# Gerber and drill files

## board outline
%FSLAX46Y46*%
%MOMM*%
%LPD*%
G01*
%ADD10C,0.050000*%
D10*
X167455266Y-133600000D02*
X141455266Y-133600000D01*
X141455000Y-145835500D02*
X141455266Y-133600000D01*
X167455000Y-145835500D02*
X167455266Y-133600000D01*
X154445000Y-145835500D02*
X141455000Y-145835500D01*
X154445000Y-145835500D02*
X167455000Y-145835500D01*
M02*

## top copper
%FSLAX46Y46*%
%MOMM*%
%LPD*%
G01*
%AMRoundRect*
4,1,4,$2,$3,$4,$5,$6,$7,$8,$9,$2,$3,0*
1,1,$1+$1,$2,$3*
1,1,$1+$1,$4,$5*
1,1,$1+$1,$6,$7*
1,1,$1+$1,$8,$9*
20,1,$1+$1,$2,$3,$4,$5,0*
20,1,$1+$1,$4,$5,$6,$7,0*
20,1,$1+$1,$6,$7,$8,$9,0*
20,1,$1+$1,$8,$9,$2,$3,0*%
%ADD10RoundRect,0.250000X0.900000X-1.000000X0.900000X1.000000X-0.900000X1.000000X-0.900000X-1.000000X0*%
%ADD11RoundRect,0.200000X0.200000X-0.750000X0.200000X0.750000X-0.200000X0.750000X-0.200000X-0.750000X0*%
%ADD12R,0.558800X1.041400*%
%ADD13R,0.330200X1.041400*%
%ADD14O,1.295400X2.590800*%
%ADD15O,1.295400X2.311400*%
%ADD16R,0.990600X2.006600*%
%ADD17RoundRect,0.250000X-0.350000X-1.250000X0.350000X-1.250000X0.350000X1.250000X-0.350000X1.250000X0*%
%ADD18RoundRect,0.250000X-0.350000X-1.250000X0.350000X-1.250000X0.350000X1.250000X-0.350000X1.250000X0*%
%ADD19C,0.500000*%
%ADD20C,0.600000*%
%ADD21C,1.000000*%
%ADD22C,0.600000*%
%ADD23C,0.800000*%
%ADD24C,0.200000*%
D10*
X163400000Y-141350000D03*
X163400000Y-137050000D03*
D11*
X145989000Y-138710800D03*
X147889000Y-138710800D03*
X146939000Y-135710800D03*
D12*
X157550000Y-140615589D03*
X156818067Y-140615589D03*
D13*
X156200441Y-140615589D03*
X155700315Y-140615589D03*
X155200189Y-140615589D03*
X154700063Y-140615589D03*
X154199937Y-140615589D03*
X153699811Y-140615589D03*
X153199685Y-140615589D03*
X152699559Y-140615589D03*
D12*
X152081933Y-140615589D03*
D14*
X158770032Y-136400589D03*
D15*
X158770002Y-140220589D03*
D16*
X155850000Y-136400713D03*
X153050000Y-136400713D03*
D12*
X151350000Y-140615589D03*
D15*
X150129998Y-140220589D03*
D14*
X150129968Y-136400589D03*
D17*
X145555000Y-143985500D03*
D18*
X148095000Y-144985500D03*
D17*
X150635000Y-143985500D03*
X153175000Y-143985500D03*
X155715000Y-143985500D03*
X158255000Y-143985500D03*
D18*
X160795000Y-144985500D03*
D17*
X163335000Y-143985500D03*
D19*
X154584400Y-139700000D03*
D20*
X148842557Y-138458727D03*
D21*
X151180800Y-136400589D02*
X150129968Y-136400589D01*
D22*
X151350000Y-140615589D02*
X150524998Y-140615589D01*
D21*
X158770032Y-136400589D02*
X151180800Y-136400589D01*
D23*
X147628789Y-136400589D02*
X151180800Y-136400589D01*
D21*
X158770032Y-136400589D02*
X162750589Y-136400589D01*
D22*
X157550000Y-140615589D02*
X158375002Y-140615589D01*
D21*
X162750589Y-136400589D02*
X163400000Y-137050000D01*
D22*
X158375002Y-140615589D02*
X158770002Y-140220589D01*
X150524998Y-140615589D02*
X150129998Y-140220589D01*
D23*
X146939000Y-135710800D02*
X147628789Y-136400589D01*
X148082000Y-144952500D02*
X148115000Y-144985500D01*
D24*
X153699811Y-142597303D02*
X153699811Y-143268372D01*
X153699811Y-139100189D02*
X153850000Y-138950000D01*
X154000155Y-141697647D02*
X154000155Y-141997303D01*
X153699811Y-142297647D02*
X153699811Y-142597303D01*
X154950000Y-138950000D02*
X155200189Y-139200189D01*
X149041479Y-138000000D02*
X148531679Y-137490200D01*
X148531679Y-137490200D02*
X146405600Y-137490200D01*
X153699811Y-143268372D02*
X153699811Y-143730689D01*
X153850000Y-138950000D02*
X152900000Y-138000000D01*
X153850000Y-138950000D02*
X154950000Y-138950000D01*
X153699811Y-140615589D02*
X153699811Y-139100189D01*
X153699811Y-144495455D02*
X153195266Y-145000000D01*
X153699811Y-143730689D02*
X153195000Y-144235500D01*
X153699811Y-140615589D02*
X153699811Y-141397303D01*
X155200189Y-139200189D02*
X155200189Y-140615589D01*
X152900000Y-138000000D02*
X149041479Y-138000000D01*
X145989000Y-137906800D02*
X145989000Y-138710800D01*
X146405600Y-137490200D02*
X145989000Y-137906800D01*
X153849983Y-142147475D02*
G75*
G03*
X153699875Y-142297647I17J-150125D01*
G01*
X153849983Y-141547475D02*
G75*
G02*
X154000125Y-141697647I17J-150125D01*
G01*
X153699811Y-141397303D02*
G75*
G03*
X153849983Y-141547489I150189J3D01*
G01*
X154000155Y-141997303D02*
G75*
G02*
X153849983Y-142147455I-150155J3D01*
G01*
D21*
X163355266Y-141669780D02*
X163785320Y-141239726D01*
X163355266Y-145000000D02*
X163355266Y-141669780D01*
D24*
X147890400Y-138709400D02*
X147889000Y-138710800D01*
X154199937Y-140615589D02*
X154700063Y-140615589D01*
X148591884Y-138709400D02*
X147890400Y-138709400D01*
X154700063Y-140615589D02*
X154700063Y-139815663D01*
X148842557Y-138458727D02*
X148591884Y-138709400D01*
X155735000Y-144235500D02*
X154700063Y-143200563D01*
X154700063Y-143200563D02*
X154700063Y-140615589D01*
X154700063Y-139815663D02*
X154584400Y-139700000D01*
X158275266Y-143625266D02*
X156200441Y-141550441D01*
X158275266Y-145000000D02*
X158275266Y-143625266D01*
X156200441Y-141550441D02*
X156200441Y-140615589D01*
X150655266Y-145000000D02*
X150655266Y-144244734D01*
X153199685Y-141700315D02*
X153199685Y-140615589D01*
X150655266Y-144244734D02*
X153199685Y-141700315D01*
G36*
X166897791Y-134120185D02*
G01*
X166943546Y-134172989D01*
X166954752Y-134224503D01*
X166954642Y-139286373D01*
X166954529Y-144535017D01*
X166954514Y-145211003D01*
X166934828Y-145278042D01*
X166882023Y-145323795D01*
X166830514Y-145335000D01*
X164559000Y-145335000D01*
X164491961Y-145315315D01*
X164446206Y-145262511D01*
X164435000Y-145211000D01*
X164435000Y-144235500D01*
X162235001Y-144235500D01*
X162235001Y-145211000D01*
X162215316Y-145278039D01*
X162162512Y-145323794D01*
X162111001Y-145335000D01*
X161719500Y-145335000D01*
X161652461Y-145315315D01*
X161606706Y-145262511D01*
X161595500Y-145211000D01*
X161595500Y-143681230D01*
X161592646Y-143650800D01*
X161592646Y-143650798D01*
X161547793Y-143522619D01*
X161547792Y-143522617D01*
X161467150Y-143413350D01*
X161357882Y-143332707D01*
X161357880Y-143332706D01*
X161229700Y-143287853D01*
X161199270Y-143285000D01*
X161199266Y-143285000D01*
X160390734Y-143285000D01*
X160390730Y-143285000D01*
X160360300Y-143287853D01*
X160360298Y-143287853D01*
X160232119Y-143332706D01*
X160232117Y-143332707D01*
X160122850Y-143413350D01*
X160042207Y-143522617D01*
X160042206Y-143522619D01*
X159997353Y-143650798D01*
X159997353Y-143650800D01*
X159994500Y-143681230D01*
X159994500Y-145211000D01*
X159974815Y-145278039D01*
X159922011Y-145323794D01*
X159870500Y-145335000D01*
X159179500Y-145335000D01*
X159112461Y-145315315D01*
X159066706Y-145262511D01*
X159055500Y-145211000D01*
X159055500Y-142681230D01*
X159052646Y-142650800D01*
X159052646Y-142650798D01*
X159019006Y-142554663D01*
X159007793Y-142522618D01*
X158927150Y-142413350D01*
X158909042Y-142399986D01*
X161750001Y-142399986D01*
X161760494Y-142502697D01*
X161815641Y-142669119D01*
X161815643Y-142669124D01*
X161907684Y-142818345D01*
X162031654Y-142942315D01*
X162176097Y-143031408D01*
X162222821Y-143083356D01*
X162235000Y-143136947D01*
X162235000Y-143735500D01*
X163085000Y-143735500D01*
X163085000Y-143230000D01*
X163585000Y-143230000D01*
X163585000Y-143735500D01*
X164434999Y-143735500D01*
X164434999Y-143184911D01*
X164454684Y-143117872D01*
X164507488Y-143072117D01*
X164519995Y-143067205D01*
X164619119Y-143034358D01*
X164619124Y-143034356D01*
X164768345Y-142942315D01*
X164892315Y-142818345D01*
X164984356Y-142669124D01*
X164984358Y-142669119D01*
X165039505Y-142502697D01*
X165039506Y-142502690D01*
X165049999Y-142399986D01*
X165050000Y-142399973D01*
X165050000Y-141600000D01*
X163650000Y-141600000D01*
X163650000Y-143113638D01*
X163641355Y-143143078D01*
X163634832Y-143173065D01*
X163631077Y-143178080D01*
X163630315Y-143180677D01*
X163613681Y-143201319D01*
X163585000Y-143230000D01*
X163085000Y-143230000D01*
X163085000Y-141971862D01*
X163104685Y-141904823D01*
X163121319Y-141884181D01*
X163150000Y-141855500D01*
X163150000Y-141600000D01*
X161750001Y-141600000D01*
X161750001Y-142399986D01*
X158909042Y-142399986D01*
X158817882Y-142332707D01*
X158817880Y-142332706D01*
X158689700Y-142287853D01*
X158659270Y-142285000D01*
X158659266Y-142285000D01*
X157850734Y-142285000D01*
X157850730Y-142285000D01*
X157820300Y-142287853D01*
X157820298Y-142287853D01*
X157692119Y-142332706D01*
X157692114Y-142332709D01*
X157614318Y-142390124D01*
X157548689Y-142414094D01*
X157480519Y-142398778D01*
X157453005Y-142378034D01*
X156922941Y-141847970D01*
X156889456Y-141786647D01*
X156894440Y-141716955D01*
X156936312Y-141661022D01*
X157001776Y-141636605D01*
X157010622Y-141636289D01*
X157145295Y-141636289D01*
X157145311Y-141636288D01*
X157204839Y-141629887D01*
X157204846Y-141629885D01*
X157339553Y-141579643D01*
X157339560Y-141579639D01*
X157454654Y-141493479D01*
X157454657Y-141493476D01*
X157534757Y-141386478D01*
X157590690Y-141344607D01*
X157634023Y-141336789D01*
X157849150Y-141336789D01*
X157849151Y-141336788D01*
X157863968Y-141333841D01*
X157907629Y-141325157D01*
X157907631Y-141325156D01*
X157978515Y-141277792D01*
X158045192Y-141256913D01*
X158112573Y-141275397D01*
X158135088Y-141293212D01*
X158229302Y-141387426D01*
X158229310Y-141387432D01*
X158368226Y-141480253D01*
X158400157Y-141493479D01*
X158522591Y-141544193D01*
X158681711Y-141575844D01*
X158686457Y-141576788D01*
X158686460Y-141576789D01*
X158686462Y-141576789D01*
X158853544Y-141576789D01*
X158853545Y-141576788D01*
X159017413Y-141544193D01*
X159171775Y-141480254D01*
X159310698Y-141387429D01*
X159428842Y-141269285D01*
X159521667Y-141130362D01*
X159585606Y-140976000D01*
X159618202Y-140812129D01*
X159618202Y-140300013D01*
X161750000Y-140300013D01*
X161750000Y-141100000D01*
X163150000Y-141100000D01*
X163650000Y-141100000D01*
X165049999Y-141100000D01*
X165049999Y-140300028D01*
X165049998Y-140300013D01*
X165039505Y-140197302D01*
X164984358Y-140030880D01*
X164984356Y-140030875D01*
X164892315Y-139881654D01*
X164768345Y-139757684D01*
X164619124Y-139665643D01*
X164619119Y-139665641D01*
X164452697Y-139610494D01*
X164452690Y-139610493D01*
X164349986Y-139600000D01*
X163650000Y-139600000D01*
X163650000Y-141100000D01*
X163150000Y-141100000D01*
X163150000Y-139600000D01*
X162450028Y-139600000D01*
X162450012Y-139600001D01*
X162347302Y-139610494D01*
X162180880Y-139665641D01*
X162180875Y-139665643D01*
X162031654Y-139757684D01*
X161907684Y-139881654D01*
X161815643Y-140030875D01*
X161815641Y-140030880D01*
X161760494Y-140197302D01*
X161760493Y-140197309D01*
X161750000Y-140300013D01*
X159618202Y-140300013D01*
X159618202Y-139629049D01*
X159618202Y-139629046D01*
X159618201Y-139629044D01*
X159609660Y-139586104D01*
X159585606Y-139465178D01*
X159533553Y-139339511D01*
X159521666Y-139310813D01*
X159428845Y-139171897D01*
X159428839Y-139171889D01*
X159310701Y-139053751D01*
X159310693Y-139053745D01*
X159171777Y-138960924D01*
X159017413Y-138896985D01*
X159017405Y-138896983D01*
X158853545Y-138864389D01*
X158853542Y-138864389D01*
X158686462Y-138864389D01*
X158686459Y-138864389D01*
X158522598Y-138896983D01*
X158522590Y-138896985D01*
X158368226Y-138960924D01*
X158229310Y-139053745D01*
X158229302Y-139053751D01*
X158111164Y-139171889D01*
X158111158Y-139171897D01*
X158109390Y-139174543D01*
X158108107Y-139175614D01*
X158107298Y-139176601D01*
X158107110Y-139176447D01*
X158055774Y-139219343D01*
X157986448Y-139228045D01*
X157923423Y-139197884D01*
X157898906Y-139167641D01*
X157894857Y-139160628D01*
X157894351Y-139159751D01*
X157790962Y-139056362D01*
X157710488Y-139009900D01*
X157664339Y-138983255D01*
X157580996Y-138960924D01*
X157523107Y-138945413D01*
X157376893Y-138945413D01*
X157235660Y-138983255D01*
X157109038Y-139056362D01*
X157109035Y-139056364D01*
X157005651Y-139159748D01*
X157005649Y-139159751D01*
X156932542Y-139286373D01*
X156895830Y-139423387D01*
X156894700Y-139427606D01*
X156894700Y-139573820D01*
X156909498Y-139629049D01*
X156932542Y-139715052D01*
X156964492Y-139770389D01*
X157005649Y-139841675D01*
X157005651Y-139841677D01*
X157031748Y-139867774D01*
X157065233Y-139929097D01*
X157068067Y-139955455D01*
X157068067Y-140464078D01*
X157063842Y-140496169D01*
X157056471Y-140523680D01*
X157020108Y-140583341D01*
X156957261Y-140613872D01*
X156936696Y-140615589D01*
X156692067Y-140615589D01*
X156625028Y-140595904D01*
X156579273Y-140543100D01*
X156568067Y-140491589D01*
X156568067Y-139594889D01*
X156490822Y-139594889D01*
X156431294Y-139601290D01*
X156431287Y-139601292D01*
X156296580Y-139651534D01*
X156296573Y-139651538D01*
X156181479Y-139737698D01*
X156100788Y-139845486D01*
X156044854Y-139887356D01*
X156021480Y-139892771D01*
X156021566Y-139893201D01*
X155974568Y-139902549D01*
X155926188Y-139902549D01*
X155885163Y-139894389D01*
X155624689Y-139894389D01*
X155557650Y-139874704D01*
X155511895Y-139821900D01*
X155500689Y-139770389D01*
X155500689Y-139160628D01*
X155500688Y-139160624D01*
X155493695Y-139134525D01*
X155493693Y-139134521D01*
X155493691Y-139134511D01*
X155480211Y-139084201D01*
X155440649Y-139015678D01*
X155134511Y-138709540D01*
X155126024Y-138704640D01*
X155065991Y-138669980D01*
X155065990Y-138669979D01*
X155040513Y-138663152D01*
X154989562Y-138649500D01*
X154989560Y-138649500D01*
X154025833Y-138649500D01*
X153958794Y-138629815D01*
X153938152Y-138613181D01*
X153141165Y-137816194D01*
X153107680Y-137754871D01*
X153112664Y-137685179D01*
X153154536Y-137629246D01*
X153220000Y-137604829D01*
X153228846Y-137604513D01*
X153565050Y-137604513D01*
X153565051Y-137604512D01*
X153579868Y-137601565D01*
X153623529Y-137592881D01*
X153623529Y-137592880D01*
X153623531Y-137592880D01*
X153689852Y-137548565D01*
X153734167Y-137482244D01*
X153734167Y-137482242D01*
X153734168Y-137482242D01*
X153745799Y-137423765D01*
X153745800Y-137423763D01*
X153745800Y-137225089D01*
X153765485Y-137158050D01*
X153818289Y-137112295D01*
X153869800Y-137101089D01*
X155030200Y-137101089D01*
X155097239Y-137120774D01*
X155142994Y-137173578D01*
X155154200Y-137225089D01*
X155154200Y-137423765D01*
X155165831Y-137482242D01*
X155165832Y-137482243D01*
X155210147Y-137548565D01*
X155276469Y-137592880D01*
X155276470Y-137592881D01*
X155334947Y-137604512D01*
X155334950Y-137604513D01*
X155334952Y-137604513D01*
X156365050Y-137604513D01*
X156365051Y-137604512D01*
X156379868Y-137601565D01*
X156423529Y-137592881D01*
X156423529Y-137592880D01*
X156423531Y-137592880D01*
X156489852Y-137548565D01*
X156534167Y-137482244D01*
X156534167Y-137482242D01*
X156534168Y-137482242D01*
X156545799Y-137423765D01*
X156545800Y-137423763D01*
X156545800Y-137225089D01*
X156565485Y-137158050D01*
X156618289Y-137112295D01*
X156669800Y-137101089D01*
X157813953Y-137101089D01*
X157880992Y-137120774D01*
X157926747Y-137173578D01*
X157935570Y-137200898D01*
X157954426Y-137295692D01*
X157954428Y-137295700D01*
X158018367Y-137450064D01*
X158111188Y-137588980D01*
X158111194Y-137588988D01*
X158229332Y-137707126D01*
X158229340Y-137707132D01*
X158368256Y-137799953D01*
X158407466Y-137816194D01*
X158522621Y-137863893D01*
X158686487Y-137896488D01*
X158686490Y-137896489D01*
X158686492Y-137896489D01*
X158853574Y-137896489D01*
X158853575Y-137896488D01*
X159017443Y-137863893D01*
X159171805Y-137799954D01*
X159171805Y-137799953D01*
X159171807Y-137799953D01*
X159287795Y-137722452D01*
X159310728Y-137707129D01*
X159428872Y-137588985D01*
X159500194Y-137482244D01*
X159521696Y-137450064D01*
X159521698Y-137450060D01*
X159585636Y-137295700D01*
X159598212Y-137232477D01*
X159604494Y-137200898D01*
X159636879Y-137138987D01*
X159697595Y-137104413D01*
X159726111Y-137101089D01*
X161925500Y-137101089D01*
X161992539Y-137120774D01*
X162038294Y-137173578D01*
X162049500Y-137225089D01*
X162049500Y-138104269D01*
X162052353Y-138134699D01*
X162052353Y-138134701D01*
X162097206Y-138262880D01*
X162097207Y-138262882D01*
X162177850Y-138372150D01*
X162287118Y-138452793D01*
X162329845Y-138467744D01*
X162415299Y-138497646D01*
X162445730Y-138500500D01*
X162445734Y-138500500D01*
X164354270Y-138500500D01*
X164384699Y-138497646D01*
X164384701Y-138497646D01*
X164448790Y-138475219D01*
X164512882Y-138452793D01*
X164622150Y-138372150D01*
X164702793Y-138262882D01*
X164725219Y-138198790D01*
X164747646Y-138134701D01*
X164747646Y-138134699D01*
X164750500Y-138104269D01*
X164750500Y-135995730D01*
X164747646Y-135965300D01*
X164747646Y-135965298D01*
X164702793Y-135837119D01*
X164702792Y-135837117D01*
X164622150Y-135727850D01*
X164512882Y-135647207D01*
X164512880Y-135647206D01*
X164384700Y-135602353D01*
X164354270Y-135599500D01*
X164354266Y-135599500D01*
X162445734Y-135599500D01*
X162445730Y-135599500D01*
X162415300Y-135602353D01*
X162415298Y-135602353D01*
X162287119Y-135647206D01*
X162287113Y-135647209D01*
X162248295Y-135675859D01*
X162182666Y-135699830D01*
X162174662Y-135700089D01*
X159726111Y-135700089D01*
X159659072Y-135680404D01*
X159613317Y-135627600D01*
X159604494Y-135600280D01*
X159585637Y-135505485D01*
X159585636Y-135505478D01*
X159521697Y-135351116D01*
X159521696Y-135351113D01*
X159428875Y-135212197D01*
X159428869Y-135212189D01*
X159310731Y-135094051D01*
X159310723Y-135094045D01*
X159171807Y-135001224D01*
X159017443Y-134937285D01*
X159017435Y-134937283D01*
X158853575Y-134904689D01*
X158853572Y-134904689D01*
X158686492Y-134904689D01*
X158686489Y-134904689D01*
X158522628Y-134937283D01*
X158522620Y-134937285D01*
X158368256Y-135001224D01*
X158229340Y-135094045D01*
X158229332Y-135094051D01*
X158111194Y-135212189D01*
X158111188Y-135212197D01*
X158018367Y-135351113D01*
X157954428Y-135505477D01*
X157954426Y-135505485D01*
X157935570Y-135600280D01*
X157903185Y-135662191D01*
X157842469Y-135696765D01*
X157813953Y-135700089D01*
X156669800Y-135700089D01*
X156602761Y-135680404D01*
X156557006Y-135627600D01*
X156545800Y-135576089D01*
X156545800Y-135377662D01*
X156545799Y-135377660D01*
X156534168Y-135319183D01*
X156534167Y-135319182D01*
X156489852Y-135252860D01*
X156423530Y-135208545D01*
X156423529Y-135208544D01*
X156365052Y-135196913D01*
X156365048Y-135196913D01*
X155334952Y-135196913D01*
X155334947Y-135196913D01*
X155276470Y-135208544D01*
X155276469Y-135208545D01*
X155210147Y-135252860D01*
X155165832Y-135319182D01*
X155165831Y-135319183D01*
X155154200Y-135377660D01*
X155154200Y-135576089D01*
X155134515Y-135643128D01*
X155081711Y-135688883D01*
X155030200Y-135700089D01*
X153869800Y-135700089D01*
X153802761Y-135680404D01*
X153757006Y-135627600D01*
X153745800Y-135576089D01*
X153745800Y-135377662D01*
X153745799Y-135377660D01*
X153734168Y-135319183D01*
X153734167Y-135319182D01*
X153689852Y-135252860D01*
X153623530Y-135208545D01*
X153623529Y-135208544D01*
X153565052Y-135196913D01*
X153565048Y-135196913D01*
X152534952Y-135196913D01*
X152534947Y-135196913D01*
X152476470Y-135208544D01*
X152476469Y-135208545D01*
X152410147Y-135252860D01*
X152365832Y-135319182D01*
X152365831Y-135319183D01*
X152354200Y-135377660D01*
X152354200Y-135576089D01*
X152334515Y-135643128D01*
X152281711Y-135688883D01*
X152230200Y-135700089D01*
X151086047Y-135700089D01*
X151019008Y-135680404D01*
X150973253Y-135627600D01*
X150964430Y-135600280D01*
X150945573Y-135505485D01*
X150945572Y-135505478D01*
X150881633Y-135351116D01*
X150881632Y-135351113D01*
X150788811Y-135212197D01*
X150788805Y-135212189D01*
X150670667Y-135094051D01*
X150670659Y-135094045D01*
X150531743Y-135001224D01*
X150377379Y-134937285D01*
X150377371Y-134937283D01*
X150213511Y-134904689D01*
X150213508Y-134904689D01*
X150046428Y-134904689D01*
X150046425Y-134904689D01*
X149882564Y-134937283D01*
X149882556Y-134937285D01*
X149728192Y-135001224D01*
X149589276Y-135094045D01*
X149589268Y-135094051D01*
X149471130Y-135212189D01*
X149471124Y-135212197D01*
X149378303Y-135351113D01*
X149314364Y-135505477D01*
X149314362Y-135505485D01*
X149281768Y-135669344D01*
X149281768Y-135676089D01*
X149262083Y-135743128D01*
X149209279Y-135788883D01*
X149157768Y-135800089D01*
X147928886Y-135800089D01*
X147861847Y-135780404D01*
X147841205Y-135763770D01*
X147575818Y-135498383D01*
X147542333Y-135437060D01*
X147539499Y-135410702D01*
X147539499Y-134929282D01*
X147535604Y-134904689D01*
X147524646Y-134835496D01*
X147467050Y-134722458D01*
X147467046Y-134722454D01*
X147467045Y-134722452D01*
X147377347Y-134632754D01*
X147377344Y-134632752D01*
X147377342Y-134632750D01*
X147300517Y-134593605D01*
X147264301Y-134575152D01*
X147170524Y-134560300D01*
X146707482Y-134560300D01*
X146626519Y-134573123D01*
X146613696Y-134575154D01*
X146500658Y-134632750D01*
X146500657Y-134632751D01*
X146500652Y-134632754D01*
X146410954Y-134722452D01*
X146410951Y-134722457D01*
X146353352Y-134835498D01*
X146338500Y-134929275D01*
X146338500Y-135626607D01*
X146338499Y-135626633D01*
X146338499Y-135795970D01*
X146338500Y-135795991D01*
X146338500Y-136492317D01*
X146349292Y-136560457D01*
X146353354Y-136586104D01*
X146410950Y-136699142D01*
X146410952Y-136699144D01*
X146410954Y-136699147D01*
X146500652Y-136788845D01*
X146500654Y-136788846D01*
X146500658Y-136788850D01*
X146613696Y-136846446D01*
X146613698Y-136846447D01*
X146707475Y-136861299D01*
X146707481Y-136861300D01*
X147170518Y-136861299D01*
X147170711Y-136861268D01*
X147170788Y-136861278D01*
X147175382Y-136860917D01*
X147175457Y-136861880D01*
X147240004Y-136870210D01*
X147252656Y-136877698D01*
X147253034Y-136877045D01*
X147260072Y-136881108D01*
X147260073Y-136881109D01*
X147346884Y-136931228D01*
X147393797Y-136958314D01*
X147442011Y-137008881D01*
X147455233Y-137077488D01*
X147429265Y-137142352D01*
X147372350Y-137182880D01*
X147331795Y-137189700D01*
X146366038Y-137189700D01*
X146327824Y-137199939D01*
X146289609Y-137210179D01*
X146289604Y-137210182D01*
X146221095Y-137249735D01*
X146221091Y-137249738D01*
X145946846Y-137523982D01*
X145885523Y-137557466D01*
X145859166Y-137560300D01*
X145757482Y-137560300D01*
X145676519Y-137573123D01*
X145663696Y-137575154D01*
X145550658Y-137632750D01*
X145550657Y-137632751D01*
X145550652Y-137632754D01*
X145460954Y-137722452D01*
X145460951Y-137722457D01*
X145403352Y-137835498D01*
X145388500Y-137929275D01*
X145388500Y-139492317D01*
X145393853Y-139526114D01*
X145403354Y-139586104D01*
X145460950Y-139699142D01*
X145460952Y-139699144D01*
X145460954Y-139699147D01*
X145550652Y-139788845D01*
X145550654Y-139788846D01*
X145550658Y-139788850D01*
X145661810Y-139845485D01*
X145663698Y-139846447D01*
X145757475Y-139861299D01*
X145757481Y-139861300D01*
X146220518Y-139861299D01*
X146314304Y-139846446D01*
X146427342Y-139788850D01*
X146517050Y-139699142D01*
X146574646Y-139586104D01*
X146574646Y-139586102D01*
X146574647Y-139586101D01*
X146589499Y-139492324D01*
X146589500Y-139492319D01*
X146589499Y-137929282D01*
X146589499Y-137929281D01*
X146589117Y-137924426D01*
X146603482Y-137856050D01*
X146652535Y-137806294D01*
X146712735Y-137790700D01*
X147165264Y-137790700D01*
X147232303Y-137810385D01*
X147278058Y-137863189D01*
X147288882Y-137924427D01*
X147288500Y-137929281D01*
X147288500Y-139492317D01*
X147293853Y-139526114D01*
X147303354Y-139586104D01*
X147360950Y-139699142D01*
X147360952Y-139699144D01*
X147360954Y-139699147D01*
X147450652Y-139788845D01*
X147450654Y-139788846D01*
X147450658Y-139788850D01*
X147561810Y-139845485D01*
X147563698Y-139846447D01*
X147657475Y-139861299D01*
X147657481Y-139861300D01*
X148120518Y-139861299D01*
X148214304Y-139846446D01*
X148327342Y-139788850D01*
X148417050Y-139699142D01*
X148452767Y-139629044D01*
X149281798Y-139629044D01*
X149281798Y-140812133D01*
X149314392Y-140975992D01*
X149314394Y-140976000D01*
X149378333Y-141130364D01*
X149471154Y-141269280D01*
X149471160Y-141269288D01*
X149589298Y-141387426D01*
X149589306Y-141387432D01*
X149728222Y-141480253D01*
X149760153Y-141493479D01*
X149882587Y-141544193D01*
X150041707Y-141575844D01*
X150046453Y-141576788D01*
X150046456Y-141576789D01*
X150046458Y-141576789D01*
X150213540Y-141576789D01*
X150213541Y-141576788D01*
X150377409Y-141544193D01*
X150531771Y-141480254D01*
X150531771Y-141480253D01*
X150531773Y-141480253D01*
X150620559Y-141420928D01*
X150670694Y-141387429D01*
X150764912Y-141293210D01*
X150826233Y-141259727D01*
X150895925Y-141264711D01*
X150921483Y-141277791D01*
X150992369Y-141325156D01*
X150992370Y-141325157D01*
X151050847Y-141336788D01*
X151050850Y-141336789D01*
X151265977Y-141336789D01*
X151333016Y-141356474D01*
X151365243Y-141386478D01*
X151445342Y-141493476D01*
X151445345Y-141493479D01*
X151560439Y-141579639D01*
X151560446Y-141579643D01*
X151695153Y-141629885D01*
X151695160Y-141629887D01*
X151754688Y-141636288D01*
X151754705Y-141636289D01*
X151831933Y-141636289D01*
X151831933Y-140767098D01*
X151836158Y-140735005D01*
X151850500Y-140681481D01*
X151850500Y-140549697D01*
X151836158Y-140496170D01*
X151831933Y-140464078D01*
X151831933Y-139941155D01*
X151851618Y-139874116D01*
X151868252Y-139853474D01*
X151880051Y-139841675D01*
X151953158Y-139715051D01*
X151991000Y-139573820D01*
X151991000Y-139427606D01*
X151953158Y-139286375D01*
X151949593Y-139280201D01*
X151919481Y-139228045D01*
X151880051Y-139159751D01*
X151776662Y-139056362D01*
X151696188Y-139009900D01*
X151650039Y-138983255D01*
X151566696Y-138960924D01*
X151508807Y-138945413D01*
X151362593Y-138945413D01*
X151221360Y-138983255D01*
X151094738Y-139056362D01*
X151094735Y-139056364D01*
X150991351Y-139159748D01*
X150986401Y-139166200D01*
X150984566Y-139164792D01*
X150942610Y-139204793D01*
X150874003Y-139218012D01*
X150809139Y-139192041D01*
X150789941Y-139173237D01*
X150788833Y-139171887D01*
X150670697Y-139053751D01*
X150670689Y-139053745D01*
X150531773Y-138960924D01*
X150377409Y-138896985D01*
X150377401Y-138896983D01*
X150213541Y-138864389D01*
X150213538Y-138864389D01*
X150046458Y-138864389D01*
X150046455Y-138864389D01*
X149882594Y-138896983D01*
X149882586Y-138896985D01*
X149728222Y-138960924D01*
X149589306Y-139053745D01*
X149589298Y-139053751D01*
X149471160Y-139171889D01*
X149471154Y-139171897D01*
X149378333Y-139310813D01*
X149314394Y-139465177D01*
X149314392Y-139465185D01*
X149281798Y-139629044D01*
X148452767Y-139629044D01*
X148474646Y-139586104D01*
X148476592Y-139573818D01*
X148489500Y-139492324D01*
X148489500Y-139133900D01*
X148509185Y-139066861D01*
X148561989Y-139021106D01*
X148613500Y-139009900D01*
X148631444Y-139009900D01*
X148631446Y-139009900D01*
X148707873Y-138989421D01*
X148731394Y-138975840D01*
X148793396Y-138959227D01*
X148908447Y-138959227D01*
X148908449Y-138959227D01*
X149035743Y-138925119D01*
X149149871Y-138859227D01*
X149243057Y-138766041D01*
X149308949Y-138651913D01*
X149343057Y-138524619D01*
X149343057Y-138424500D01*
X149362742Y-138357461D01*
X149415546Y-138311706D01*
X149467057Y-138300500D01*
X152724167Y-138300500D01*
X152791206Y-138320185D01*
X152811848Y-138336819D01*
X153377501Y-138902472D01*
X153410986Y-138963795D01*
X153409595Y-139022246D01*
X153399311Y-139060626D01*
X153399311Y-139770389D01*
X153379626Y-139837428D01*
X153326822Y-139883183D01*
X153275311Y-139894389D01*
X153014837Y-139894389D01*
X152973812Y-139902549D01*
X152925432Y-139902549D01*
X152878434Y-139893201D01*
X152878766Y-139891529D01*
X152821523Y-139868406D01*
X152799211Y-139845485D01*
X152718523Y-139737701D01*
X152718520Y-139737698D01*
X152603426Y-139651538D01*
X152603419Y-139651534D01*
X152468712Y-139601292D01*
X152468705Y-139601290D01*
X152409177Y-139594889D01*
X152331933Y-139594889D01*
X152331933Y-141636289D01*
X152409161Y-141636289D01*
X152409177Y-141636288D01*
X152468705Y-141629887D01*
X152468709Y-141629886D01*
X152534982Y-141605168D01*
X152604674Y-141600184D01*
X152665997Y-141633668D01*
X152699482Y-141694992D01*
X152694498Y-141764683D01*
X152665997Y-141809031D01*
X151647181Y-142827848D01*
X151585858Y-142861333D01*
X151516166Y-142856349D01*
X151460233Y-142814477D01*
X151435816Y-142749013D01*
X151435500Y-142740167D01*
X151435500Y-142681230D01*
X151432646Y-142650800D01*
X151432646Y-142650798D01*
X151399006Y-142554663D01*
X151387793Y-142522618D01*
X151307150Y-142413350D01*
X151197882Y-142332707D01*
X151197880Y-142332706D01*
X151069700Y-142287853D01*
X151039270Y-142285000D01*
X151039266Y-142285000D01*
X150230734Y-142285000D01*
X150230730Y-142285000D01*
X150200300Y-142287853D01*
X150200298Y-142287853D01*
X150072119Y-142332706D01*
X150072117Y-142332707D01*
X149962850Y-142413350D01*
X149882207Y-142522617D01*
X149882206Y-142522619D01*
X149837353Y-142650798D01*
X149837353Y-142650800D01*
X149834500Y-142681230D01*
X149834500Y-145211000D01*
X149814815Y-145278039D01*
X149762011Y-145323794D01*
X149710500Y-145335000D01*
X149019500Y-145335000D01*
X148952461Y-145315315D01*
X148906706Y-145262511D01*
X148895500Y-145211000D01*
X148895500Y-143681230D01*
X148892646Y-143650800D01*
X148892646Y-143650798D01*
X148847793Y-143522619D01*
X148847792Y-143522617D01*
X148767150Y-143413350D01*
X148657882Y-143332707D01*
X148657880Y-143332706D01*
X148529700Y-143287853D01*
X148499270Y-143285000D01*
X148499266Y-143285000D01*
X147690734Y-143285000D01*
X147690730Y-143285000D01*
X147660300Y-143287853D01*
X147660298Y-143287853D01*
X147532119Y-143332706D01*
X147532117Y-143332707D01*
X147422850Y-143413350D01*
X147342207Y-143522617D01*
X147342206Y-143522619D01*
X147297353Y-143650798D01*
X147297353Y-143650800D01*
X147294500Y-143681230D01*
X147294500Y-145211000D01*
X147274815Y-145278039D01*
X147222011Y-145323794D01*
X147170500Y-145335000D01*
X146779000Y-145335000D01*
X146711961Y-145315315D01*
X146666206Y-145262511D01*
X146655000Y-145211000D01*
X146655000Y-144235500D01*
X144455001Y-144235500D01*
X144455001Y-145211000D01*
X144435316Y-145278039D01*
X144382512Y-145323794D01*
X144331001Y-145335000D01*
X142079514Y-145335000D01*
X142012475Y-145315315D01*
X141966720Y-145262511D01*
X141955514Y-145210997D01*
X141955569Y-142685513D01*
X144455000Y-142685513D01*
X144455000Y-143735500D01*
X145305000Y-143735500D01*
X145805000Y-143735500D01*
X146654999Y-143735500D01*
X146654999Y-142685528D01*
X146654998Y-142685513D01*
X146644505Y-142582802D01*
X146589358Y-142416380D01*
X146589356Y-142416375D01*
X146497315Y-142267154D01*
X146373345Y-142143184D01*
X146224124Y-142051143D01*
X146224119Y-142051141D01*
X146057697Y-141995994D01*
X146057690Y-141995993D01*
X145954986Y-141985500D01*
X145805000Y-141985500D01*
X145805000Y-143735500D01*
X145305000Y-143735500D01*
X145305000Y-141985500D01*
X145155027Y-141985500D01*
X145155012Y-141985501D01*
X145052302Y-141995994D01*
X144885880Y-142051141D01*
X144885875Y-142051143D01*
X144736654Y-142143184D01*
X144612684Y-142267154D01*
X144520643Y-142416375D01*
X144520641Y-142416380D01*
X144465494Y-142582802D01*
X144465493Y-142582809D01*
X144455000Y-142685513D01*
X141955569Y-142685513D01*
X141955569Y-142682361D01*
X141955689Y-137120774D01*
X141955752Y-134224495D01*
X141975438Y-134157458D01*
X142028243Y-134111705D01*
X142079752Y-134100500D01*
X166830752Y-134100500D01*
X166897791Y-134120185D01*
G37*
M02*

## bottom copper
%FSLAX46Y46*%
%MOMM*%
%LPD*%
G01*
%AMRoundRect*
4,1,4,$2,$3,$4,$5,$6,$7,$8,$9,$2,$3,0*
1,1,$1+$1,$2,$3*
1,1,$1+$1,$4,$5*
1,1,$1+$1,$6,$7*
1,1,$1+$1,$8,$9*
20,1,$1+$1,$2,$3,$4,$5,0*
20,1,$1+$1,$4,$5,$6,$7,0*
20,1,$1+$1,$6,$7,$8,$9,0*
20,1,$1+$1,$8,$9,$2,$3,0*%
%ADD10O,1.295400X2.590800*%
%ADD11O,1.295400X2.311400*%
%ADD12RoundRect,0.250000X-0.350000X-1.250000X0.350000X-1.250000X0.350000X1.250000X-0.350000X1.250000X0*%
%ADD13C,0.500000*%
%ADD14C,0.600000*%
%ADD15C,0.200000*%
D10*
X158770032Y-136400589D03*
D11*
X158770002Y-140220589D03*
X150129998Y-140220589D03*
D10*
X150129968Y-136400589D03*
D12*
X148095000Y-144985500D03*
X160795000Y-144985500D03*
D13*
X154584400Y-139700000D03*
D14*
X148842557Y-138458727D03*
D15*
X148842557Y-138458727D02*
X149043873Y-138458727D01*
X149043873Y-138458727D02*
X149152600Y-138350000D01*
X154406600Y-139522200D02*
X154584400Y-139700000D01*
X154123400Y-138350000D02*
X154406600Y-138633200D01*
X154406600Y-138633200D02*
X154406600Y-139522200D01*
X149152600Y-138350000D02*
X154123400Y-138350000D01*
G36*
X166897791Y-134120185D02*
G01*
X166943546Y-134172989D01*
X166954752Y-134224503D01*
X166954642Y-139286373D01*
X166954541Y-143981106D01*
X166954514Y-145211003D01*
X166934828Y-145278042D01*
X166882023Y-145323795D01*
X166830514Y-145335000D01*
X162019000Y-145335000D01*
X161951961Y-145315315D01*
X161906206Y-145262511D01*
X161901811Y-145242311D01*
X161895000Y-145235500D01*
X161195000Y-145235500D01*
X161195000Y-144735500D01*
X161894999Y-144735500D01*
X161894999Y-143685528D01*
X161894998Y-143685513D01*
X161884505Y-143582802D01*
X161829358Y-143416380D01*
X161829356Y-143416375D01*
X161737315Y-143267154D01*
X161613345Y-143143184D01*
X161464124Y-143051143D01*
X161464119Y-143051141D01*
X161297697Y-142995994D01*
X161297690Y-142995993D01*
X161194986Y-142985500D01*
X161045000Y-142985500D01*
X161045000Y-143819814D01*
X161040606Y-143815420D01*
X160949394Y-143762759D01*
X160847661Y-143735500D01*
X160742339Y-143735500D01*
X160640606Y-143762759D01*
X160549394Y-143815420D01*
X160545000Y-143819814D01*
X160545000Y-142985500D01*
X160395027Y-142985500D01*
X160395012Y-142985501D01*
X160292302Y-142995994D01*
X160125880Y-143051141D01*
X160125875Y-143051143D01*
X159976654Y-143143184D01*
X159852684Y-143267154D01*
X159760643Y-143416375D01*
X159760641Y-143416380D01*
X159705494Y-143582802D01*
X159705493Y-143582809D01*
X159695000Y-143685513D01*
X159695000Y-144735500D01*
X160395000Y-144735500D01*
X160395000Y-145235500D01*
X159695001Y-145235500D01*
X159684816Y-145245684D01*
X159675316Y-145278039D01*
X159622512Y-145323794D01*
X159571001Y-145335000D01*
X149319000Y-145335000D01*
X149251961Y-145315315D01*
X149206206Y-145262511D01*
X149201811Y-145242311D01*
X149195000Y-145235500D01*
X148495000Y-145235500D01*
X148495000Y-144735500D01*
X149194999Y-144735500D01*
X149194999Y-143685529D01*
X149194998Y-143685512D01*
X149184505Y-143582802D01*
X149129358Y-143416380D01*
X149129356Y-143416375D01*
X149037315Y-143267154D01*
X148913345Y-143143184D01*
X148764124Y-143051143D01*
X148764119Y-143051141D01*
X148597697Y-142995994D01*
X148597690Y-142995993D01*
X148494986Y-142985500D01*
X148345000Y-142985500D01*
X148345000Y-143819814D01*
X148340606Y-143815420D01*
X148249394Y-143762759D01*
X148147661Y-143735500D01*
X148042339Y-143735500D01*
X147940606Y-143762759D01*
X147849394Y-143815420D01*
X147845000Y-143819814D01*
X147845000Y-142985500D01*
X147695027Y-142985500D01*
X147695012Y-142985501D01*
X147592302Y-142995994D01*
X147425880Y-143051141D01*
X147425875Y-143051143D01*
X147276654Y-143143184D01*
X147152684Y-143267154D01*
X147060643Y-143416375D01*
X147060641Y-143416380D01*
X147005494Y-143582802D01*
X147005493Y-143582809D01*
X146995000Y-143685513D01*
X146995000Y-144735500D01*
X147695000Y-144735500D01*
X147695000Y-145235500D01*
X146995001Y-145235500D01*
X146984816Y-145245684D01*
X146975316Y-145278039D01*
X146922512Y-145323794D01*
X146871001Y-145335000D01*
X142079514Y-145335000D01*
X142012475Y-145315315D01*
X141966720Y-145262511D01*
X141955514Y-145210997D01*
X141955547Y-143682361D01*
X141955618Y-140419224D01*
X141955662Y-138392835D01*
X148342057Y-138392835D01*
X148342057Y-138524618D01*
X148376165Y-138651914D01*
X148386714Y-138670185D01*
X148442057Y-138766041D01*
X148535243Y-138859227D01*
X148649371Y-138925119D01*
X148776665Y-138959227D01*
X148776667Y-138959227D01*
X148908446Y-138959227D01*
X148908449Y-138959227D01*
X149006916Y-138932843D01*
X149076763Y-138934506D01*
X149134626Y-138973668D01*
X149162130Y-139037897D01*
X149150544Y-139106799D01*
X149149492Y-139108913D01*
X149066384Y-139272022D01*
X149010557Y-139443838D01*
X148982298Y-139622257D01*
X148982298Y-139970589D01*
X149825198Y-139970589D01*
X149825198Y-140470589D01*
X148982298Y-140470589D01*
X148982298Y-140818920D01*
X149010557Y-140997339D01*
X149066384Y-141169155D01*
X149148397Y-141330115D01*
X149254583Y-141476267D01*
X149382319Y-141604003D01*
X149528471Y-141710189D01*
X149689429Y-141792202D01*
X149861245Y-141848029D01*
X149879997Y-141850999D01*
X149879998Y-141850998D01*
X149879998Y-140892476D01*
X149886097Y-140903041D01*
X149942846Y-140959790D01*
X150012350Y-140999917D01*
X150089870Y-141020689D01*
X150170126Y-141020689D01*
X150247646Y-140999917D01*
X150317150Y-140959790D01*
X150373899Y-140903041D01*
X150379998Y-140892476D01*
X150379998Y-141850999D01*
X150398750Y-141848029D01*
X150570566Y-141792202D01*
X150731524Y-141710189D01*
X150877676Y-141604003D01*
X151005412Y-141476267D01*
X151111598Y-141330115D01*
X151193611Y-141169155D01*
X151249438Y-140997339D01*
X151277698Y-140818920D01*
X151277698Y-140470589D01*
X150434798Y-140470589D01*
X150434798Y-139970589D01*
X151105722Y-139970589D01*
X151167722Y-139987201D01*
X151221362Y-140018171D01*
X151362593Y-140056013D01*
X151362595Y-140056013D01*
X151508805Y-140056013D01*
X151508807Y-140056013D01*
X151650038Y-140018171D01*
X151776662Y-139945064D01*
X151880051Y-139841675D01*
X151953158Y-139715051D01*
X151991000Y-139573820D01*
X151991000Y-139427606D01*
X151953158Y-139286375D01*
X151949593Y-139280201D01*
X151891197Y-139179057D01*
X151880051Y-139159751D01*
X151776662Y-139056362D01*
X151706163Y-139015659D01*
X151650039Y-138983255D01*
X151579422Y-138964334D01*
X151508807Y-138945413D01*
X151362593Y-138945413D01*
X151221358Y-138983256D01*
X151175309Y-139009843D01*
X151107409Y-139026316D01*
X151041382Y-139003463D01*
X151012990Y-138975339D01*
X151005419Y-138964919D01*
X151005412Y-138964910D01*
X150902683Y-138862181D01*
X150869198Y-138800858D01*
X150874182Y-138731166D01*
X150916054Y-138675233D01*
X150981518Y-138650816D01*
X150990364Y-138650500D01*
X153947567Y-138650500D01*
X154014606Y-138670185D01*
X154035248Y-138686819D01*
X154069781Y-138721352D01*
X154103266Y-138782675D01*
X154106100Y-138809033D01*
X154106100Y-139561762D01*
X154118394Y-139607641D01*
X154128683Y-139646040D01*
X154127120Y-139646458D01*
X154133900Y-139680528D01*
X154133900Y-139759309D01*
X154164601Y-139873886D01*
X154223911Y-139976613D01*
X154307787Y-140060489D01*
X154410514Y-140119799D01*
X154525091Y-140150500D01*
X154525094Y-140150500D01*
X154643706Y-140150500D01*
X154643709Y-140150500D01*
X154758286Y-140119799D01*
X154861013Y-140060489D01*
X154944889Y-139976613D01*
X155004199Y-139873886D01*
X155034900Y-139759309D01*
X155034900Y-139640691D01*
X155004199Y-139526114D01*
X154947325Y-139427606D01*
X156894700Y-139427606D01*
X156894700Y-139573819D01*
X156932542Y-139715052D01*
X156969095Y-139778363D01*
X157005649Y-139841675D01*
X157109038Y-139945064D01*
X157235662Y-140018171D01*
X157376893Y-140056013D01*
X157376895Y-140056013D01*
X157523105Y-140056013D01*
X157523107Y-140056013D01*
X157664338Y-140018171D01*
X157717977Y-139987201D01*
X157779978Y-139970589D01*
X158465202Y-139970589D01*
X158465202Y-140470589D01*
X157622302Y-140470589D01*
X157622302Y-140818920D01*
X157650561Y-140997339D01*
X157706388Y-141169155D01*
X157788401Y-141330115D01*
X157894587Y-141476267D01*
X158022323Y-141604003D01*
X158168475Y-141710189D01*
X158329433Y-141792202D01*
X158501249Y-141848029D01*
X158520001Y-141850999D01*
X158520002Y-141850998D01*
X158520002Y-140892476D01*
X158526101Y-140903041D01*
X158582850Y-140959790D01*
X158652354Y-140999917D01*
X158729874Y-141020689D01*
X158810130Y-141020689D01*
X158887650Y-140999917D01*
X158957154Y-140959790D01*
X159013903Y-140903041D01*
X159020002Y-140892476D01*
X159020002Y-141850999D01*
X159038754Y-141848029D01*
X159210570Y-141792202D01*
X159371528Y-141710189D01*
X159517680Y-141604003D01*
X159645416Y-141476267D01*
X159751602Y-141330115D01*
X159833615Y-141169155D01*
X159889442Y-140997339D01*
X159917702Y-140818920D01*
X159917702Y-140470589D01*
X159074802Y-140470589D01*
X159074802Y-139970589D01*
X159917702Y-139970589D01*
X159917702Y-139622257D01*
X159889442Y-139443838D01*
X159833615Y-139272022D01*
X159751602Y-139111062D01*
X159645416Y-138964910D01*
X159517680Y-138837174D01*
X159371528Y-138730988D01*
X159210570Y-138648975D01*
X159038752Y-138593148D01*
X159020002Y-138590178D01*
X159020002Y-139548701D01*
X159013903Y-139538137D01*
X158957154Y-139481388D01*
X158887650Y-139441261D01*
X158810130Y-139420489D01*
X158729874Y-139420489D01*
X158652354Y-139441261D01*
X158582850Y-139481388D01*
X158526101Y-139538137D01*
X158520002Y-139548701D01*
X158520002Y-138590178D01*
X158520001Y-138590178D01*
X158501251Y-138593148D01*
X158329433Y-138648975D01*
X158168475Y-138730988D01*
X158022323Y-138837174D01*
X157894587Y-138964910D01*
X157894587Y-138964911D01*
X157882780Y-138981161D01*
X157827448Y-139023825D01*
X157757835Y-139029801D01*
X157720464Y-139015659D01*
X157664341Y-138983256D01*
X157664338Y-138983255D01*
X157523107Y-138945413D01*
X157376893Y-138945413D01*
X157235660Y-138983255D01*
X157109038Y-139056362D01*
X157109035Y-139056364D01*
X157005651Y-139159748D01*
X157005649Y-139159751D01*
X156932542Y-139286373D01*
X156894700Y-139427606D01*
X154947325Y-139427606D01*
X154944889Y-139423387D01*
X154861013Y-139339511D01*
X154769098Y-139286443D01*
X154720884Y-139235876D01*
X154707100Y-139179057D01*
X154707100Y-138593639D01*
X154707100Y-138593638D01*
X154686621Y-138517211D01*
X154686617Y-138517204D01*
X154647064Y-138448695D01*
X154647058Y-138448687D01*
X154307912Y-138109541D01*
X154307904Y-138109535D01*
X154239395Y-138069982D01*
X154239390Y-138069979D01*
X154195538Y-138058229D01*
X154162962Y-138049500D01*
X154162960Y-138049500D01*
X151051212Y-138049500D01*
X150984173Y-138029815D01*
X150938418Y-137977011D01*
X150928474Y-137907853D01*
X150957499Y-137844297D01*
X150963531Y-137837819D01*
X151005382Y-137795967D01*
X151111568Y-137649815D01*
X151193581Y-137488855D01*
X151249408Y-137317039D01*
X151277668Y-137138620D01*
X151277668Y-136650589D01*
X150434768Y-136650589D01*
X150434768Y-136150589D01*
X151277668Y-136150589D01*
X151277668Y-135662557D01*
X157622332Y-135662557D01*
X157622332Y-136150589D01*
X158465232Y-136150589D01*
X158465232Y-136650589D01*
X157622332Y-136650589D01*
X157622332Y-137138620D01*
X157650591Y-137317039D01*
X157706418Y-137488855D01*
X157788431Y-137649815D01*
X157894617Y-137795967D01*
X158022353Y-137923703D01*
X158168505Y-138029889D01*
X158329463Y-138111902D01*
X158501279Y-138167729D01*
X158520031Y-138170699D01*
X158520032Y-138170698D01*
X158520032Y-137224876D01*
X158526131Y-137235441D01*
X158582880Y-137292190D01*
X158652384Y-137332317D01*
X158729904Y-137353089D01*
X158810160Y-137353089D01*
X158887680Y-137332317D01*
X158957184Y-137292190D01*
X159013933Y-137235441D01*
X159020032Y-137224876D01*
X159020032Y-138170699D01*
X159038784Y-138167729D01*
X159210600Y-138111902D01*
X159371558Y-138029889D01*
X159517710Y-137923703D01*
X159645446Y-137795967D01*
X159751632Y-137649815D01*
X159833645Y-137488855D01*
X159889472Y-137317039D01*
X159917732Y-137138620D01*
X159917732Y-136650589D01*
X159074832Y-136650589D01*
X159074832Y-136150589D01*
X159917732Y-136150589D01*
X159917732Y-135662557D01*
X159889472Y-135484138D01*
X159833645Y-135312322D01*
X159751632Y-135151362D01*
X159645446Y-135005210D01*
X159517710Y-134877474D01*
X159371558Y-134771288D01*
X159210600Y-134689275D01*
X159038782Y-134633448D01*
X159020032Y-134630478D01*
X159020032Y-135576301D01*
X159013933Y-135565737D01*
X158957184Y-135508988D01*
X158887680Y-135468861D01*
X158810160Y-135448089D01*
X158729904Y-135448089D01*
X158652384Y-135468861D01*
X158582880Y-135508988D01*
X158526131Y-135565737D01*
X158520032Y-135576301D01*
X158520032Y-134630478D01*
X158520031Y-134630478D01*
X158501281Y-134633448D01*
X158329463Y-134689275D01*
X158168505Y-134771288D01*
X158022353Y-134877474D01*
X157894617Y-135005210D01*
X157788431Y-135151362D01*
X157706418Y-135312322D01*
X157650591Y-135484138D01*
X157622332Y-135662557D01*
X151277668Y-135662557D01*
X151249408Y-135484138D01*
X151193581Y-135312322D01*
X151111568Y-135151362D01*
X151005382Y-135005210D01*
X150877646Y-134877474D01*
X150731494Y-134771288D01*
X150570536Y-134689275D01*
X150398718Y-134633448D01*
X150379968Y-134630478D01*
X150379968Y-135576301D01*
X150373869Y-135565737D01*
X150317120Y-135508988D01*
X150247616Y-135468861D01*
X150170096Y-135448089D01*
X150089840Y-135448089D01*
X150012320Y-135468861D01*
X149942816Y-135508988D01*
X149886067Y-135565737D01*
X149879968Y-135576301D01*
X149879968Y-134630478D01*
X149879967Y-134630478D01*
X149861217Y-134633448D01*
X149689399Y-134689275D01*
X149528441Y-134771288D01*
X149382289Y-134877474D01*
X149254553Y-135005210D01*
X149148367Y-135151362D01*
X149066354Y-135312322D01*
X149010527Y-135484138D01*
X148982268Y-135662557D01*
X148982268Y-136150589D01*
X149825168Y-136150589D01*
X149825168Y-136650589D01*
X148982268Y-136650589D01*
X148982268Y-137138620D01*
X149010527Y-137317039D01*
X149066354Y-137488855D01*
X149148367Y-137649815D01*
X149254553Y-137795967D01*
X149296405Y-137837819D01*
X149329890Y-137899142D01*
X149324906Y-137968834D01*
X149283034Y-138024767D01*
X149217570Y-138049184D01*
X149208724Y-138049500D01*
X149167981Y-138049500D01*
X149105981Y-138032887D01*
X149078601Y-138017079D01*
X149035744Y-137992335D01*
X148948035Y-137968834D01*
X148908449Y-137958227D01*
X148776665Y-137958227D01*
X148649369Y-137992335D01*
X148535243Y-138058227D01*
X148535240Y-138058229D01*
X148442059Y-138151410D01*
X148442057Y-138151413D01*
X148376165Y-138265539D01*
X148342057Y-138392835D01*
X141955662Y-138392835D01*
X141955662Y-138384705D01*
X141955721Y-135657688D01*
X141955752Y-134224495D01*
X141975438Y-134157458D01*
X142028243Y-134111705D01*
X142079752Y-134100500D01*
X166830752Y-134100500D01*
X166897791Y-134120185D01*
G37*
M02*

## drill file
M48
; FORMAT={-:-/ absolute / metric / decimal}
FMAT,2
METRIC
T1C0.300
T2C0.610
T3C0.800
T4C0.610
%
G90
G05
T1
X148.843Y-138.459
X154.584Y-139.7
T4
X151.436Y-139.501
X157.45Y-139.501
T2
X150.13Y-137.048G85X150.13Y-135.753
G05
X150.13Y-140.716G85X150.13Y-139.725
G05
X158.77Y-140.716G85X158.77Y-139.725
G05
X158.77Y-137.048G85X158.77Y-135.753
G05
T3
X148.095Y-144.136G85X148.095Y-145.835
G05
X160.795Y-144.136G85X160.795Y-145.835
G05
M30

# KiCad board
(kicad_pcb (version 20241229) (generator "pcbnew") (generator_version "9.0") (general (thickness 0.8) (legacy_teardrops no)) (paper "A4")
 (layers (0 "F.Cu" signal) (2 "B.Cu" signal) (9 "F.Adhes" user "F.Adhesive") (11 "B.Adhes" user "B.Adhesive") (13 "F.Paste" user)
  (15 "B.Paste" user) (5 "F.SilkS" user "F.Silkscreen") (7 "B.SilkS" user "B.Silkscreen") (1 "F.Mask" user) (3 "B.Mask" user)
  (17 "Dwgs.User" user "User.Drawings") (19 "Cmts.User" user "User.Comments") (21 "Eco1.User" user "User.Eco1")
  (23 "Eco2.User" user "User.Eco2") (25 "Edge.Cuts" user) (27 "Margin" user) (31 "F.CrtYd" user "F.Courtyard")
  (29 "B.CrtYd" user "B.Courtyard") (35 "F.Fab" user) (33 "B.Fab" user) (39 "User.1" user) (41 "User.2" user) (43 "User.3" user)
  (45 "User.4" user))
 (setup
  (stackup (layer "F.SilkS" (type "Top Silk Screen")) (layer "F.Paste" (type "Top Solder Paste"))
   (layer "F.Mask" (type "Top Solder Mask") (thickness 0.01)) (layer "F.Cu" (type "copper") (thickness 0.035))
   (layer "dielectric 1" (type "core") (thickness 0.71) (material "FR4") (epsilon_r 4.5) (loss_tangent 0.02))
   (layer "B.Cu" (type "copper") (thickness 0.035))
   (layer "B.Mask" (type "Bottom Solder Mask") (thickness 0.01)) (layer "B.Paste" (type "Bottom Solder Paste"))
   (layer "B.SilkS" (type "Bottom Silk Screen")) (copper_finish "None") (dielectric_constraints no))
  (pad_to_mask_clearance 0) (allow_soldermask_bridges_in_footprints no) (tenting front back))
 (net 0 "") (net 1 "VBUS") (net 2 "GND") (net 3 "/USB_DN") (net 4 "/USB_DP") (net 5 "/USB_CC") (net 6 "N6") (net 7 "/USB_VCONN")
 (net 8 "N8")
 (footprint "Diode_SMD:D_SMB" (layer "F.Cu") (at 163.4 139.2 90)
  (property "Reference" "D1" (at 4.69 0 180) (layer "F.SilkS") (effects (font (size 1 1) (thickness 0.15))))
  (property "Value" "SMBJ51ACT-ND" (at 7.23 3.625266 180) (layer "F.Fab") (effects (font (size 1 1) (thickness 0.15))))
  (pad "1" smd roundrect (at -2.15 0 90) (size 2.5 2.3) (layers "F.Cu" "F.Mask" "F.Paste") (roundrect_rratio 0.1086956522) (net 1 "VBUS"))
  (pad "2" smd roundrect (at 2.15 0 90) (size 2.5 2.3) (layers "F.Cu" "F.Mask" "F.Paste") (roundrect_rratio 0.1086956522) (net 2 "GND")))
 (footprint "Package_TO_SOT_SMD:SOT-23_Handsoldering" (layer "F.Cu") (at 146.939 137.2108 90)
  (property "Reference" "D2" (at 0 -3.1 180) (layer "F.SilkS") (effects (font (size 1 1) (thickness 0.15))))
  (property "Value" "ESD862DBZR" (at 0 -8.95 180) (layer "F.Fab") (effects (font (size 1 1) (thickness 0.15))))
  (pad "1" smd roundrect (at -1.5 -0.95 90) (size 1.9 0.8) (layers "F.Cu" "F.Mask" "F.Paste") (roundrect_rratio 0.25) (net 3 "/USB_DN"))
  (pad "2" smd roundrect (at -1.5 0.95 90) (size 1.9 0.8) (layers "F.Cu" "F.Mask" "F.Paste") (roundrect_rratio 0.25) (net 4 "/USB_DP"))
  (pad "3" smd roundrect (at 1.5 0 90) (size 1.9 0.8) (layers "F.Cu" "F.Mask" "F.Paste") (roundrect_rratio 0.25) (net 2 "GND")))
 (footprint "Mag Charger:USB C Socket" (layer "F.Cu") (at 154.45 137.4 180)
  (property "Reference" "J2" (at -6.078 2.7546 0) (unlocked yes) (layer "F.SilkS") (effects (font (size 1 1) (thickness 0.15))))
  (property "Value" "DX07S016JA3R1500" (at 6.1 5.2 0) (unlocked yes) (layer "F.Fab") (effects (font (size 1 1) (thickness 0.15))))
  (pad "" np_thru_hole circle (at -3 -2.100713 180) (size 0.6096 0.6096) (drill 0.6096) (layers))
  (pad "" np_thru_hole circle (at 3.0143 -2.100713 180) (size 0.6096 0.6096) (drill 0.6096) (layers))
  (pad "1" smd rect (at -3.1 -3.215589 180) (size 0.5588 1.0414) (layers "F.Cu" "F.Mask" "F.Paste") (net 2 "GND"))
  (pad "2" smd rect (at -2.368067 -3.215589 180) (size 0.5588 1.0414) (layers "F.Cu" "F.Mask" "F.Paste") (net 1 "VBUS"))
  (pad "3" smd rect (at -1.750441 -3.215589 180) (size 0.3302 1.0414) (layers "F.Cu" "F.Mask" "F.Paste") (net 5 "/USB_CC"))
  (pad "4" smd rect (at -1.250315 -3.215589 180) (size 0.3302 1.0414) (layers "F.Cu" "F.Mask" "F.Paste") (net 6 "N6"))
  (pad "5" smd rect (at -0.750189 -3.215589 180) (size 0.3302 1.0414) (layers "F.Cu" "F.Mask" "F.Paste") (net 3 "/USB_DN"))
  (pad "6" smd rect (at -0.250063 -3.215589 180) (size 0.3302 1.0414) (layers "F.Cu" "F.Mask" "F.Paste") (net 4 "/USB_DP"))
  (pad "7" smd rect (at 0.250063 -3.215589 180) (size 0.3302 1.0414) (layers "F.Cu" "F.Mask" "F.Paste") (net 4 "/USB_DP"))
  (pad "8" smd rect (at 0.750189 -3.215589 180) (size 0.3302 1.0414) (layers "F.Cu" "F.Mask" "F.Paste") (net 3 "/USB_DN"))
  (pad "9" smd rect (at 1.250315 -3.215589 180) (size 0.3302 1.0414) (layers "F.Cu" "F.Mask" "F.Paste") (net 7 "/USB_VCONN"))
  (pad "10" smd rect (at 1.750441 -3.215589 180) (size 0.3302 1.0414) (layers "F.Cu" "F.Mask" "F.Paste") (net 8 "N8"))
  (pad "11" smd rect (at 2.368067 -3.215589 180) (size 0.5588 1.0414) (layers "F.Cu" "F.Mask" "F.Paste") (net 1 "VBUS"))
  (pad "12" thru_hole oval (at -4.320032 0.999411 180) (size 1.2954 2.5908) (drill oval 0.6096 1.905) (layers "*.Cu" "*.Mask")
   (remove_unused_layers no) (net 2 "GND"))
  (pad "12" thru_hole oval (at -4.320002 -2.820589 180) (size 1.2954 2.3114) (drill oval 0.6096 1.6002) (layers "*.Cu" "*.Mask")
   (remove_unused_layers no) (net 2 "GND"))
  (pad "12" smd rect (at -1.4 0.999287 180) (size 0.9906 2.0066) (layers "F.Cu" "F.Mask" "F.Paste") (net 2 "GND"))
  (pad "12" smd rect (at 1.4 0.999287 180) (size 0.9906 2.0066) (layers "F.Cu" "F.Mask" "F.Paste") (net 2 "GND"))
  (pad "12" smd rect (at 3.1 -3.215589 180) (size 0.5588 1.0414) (layers "F.Cu" "F.Mask" "F.Paste") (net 2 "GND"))
  (pad "12" thru_hole oval (at 4.320002 -2.820589 180) (size 1.2954 2.3114) (drill oval 0.6096 1.6002) (layers "*.Cu" "*.Mask")
   (remove_unused_layers no) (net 2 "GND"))
  (pad "12" thru_hole oval (at 4.320032 0.999411 180) (size 1.2954 2.5908) (drill oval 0.6096 1.905) (layers "*.Cu" "*.Mask")
   (remove_unused_layers no) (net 2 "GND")))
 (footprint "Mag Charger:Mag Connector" (layer "F.Cu") (at 154.445 143.3345)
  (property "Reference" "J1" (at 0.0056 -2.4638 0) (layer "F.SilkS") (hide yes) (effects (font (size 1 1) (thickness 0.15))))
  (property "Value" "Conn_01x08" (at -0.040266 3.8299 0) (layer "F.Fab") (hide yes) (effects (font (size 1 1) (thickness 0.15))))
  (fp_line (start 0 2.501) (end -12.99 2.501) (stroke (width 0.05) (type default)) (layer "Edge.Cuts"))
  (fp_line (start 0 2.501) (end 13.01 2.501) (stroke (width 0.05) (type default)) (layer "Edge.Cuts"))
  (pad "1" smd roundrect (at -8.89 0.651) (size 1.2 3) (layers "F.Cu" "F.Mask" "F.Paste") (roundrect_rratio 0.2083333333) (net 1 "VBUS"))
  (pad "2" thru_hole roundrect (at -6.35 1.651) (size 1.2 3) (drill oval 0.8 2.5) (layers "*.Cu" "*.Mask") (remove_unused_layers no)
   (roundrect_rratio 0.2083333333) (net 2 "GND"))
  (pad "3" smd roundrect (at -3.81 0.651) (size 1.2 3) (layers "F.Cu" "F.Mask" "F.Paste") (roundrect_rratio 0.2083333333)
   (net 7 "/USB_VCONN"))
  (pad "4" smd roundrect (at -1.27 0.651) (size 1.2 3) (layers "F.Cu" "F.Mask" "F.Paste") (roundrect_rratio 0.2083333333) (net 3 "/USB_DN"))
  (pad "5" smd roundrect (at 1.27 0.651) (size 1.2 3) (layers "F.Cu" "F.Mask" "F.Paste") (roundrect_rratio 0.2083333333) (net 4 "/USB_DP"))
  (pad "6" smd roundrect (at 3.81 0.651) (size 1.2 3) (layers "F.Cu" "F.Mask" "F.Paste") (roundrect_rratio 0.2083333333) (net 5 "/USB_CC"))
  (pad "7" thru_hole roundrect (at 6.35 1.651) (size 1.2 3) (drill oval 0.8 2.5) (layers "*.Cu" "*.Mask") (remove_unused_layers no)
   (roundrect_rratio 0.2083333333) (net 2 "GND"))
  (pad "8" smd roundrect (at 8.89 0.651) (size 1.2 3) (layers "F.Cu" "F.Mask" "F.Paste") (roundrect_rratio 0.2083333333) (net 1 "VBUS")))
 (gr_line (start 167.455266 133.6) (end 141.455266 133.6) (stroke (width 0.05) (type default)) (layer "Edge.Cuts"))
 (gr_line (start 141.455 145.8355) (end 141.455266 133.6) (stroke (width 0.05) (type default)) (layer "Edge.Cuts"))
 (gr_line (start 167.455 145.8355) (end 167.455266 133.6) (stroke (width 0.05) (type default)) (layer "Edge.Cuts"))
 (segment (start 151.1808 136.400589) (end 150.129968 136.400589) (width 1) (layer "F.Cu") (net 2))
 (segment (start 151.35 140.615589) (end 150.524998 140.615589) (width 0.6) (layer "F.Cu") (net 2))
 (segment (start 158.770032 136.400589) (end 151.1808 136.400589) (width 1) (layer "F.Cu") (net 2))
 (segment (start 147.628789 136.400589) (end 151.1808 136.400589) (width 0.8) (layer "F.Cu") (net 2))
 (segment (start 158.770032 136.400589) (end 162.750589 136.400589) (width 1) (layer "F.Cu") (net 2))
 (segment (start 157.55 140.615589) (end 158.375002 140.615589) (width 0.6) (layer "F.Cu") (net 2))
 (segment (start 162.750589 136.400589) (end 163.4 137.05) (width 1) (layer "F.Cu") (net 2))
 (segment (start 158.375002 140.615589) (end 158.770002 140.220589) (width 0.6) (layer "F.Cu") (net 2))
 (segment (start 150.524998 140.615589) (end 150.129998 140.220589) (width 0.6) (layer "F.Cu") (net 2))
 (segment (start 146.939 135.7108) (end 147.628789 136.400589) (width 0.8) (layer "F.Cu") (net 2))
 (segment (start 148.082 144.9525) (end 148.115 144.9855) (width 0.8) (layer "F.Cu") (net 2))
 (segment (start 153.699811 142.597303) (end 153.699811 143.268372) (width 0.2) (layer "F.Cu") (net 3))
 (segment (start 153.699811 139.100189) (end 153.85 138.95) (width 0.2) (layer "F.Cu") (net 3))
 (segment (start 154.000155 141.697647) (end 154.000155 141.997303) (width 0.2) (layer "F.Cu") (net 3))
 (segment (start 153.699811 142.297647) (end 153.699811 142.597303) (width 0.2) (layer "F.Cu") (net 3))
 (segment (start 154.95 138.95) (end 155.200189 139.200189) (width 0.2) (layer "F.Cu") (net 3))
 (segment (start 149.041479 138) (end 148.531679 137.4902) (width 0.2) (layer "F.Cu") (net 3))
 (segment (start 148.531679 137.4902) (end 146.4056 137.4902) (width 0.2) (layer "F.Cu") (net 3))
 (segment (start 153.699811 143.268372) (end 153.699811 143.730689) (width 0.2) (layer "F.Cu") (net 3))
 (segment (start 153.85 138.95) (end 152.9 138) (width 0.2) (layer "F.Cu") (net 3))
 (segment (start 153.85 138.95) (end 154.95 138.95) (width 0.2) (layer "F.Cu") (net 3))
 (segment (start 153.699811 140.615589) (end 153.699811 139.100189) (width 0.2) (layer "F.Cu") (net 3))
 (segment (start 153.699811 144.495455) (end 153.195266 145) (width 0.2) (layer "F.Cu") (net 3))
 (segment (start 153.699811 143.730689) (end 153.195 144.2355) (width 0.2) (layer "F.Cu") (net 3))
 (segment (start 153.699811 140.615589) (end 153.699811 141.397303) (width 0.2) (layer "F.Cu") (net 3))
 (segment (start 155.200189 139.200189) (end 155.200189 140.615589) (width 0.2) (layer "F.Cu") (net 3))
 (segment (start 152.9 138) (end 149.041479 138) (width 0.2) (layer "F.Cu") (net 3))
 (segment (start 145.989 137.9068) (end 145.989 138.7108) (width 0.2) (layer "F.Cu") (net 3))
 (segment (start 146.4056 137.4902) (end 145.989 137.9068) (width 0.2) (layer "F.Cu") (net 3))
 (arc (start 153.849983 142.147475) (mid 153.743795 142.191459) (end 153.699811 142.297647) (width 0.2) (layer "F.Cu") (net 3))
 (arc (start 153.849983 141.547475) (mid 153.956171 141.591459) (end 154.000155 141.697647) (width 0.2) (layer "F.Cu") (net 3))
 (arc (start 153.699811 141.397303) (mid 153.743795 141.503491) (end 153.849983 141.547475) (width 0.2) (layer "F.Cu") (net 3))
 (arc (start 154.000155 141.997303) (mid 153.956171 142.103491) (end 153.849983 142.147475) (width 0.2) (layer "F.Cu") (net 3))
 (segment (start 163.355266 141.66978) (end 163.78532 141.239726) (width 1) (layer "F.Cu") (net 1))
 (segment (start 163.355266 145) (end 163.355266 141.66978) (width 1) (layer "F.Cu") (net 1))
 (segment (start 147.8904 138.7094) (end 147.889 138.7108) (width 0.2) (layer "F.Cu") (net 4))
 (segment (start 154.199937 140.615589) (end 154.700063 140.615589) (width 0.2) (layer "F.Cu") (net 4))
 (segment (start 148.591884 138.7094) (end 147.8904 138.7094) (width 0.2) (layer "F.Cu") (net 4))
 (segment (start 154.700063 140.615589) (end 154.700063 139.815663) (width 0.2) (layer "F.Cu") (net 4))
 (segment (start 148.842557 138.458727) (end 148.591884 138.7094) (width 0.2) (layer "F.Cu") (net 4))
 (segment (start 155.735 144.2355) (end 154.700063 143.200563) (width 0.2) (layer "F.Cu") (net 4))
 (segment (start 154.700063 143.200563) (end 154.700063 140.615589) (width 0.2) (layer "F.Cu") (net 4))
 (segment (start 154.700063 139.815663) (end 154.5844 139.7) (width 0.2) (layer "F.Cu") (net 4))
 (via (at 154.5844 139.7) (size 0.5) (drill 0.3) (layers "F.Cu" "B.Cu") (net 4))
 (via (at 148.842557 138.458727) (size 0.6) (drill 0.3) (layers "F.Cu" "B.Cu") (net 4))
 (segment (start 148.842557 138.458727) (end 149.043873 138.458727) (width 0.2) (layer "B.Cu") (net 4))
 (segment (start 149.043873 138.458727) (end 149.1526 138.35) (width 0.2) (layer "B.Cu") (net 4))
 (segment (start 154.4066 139.5222) (end 154.5844 139.7) (width 0.2) (layer "B.Cu") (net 4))
 (segment (start 154.1234 138.35) (end 154.4066 138.6332) (width 0.2) (layer "B.Cu") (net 4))
 (segment (start 154.4066 138.6332) (end 154.4066 139.5222) (width 0.2) (layer "B.Cu") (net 4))
 (segment (start 149.1526 138.35) (end 154.1234 138.35) (width 0.2) (layer "B.Cu") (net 4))
 (segment (start 158.275266 143.625266) (end 156.200441 141.550441) (width 0.2) (layer "F.Cu") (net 5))
 (segment (start 158.275266 145) (end 158.275266 143.625266) (width 0.2) (layer "F.Cu") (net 5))
 (segment (start 156.200441 141.550441) (end 156.200441 140.615589) (width 0.2) (layer "F.Cu") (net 5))
 (segment (start 150.655266 145) (end 150.655266 144.244734) (width 0.2) (layer "F.Cu") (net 7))
 (segment (start 153.199685 141.700315) (end 153.199685 140.615589) (width 0.2) (layer "F.Cu") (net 7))
 (segment (start 150.655266 144.244734) (end 153.199685 141.700315) (width 0.2) (layer "F.Cu") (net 7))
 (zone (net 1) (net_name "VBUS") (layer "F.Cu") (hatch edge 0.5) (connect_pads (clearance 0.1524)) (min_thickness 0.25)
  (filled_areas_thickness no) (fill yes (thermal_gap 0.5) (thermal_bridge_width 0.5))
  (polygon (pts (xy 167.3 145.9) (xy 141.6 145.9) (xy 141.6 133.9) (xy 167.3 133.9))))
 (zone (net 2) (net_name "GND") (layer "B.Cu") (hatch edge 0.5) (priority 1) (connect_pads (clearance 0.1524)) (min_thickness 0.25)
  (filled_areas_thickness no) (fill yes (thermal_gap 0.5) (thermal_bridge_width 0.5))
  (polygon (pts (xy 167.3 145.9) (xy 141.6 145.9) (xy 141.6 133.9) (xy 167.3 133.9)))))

